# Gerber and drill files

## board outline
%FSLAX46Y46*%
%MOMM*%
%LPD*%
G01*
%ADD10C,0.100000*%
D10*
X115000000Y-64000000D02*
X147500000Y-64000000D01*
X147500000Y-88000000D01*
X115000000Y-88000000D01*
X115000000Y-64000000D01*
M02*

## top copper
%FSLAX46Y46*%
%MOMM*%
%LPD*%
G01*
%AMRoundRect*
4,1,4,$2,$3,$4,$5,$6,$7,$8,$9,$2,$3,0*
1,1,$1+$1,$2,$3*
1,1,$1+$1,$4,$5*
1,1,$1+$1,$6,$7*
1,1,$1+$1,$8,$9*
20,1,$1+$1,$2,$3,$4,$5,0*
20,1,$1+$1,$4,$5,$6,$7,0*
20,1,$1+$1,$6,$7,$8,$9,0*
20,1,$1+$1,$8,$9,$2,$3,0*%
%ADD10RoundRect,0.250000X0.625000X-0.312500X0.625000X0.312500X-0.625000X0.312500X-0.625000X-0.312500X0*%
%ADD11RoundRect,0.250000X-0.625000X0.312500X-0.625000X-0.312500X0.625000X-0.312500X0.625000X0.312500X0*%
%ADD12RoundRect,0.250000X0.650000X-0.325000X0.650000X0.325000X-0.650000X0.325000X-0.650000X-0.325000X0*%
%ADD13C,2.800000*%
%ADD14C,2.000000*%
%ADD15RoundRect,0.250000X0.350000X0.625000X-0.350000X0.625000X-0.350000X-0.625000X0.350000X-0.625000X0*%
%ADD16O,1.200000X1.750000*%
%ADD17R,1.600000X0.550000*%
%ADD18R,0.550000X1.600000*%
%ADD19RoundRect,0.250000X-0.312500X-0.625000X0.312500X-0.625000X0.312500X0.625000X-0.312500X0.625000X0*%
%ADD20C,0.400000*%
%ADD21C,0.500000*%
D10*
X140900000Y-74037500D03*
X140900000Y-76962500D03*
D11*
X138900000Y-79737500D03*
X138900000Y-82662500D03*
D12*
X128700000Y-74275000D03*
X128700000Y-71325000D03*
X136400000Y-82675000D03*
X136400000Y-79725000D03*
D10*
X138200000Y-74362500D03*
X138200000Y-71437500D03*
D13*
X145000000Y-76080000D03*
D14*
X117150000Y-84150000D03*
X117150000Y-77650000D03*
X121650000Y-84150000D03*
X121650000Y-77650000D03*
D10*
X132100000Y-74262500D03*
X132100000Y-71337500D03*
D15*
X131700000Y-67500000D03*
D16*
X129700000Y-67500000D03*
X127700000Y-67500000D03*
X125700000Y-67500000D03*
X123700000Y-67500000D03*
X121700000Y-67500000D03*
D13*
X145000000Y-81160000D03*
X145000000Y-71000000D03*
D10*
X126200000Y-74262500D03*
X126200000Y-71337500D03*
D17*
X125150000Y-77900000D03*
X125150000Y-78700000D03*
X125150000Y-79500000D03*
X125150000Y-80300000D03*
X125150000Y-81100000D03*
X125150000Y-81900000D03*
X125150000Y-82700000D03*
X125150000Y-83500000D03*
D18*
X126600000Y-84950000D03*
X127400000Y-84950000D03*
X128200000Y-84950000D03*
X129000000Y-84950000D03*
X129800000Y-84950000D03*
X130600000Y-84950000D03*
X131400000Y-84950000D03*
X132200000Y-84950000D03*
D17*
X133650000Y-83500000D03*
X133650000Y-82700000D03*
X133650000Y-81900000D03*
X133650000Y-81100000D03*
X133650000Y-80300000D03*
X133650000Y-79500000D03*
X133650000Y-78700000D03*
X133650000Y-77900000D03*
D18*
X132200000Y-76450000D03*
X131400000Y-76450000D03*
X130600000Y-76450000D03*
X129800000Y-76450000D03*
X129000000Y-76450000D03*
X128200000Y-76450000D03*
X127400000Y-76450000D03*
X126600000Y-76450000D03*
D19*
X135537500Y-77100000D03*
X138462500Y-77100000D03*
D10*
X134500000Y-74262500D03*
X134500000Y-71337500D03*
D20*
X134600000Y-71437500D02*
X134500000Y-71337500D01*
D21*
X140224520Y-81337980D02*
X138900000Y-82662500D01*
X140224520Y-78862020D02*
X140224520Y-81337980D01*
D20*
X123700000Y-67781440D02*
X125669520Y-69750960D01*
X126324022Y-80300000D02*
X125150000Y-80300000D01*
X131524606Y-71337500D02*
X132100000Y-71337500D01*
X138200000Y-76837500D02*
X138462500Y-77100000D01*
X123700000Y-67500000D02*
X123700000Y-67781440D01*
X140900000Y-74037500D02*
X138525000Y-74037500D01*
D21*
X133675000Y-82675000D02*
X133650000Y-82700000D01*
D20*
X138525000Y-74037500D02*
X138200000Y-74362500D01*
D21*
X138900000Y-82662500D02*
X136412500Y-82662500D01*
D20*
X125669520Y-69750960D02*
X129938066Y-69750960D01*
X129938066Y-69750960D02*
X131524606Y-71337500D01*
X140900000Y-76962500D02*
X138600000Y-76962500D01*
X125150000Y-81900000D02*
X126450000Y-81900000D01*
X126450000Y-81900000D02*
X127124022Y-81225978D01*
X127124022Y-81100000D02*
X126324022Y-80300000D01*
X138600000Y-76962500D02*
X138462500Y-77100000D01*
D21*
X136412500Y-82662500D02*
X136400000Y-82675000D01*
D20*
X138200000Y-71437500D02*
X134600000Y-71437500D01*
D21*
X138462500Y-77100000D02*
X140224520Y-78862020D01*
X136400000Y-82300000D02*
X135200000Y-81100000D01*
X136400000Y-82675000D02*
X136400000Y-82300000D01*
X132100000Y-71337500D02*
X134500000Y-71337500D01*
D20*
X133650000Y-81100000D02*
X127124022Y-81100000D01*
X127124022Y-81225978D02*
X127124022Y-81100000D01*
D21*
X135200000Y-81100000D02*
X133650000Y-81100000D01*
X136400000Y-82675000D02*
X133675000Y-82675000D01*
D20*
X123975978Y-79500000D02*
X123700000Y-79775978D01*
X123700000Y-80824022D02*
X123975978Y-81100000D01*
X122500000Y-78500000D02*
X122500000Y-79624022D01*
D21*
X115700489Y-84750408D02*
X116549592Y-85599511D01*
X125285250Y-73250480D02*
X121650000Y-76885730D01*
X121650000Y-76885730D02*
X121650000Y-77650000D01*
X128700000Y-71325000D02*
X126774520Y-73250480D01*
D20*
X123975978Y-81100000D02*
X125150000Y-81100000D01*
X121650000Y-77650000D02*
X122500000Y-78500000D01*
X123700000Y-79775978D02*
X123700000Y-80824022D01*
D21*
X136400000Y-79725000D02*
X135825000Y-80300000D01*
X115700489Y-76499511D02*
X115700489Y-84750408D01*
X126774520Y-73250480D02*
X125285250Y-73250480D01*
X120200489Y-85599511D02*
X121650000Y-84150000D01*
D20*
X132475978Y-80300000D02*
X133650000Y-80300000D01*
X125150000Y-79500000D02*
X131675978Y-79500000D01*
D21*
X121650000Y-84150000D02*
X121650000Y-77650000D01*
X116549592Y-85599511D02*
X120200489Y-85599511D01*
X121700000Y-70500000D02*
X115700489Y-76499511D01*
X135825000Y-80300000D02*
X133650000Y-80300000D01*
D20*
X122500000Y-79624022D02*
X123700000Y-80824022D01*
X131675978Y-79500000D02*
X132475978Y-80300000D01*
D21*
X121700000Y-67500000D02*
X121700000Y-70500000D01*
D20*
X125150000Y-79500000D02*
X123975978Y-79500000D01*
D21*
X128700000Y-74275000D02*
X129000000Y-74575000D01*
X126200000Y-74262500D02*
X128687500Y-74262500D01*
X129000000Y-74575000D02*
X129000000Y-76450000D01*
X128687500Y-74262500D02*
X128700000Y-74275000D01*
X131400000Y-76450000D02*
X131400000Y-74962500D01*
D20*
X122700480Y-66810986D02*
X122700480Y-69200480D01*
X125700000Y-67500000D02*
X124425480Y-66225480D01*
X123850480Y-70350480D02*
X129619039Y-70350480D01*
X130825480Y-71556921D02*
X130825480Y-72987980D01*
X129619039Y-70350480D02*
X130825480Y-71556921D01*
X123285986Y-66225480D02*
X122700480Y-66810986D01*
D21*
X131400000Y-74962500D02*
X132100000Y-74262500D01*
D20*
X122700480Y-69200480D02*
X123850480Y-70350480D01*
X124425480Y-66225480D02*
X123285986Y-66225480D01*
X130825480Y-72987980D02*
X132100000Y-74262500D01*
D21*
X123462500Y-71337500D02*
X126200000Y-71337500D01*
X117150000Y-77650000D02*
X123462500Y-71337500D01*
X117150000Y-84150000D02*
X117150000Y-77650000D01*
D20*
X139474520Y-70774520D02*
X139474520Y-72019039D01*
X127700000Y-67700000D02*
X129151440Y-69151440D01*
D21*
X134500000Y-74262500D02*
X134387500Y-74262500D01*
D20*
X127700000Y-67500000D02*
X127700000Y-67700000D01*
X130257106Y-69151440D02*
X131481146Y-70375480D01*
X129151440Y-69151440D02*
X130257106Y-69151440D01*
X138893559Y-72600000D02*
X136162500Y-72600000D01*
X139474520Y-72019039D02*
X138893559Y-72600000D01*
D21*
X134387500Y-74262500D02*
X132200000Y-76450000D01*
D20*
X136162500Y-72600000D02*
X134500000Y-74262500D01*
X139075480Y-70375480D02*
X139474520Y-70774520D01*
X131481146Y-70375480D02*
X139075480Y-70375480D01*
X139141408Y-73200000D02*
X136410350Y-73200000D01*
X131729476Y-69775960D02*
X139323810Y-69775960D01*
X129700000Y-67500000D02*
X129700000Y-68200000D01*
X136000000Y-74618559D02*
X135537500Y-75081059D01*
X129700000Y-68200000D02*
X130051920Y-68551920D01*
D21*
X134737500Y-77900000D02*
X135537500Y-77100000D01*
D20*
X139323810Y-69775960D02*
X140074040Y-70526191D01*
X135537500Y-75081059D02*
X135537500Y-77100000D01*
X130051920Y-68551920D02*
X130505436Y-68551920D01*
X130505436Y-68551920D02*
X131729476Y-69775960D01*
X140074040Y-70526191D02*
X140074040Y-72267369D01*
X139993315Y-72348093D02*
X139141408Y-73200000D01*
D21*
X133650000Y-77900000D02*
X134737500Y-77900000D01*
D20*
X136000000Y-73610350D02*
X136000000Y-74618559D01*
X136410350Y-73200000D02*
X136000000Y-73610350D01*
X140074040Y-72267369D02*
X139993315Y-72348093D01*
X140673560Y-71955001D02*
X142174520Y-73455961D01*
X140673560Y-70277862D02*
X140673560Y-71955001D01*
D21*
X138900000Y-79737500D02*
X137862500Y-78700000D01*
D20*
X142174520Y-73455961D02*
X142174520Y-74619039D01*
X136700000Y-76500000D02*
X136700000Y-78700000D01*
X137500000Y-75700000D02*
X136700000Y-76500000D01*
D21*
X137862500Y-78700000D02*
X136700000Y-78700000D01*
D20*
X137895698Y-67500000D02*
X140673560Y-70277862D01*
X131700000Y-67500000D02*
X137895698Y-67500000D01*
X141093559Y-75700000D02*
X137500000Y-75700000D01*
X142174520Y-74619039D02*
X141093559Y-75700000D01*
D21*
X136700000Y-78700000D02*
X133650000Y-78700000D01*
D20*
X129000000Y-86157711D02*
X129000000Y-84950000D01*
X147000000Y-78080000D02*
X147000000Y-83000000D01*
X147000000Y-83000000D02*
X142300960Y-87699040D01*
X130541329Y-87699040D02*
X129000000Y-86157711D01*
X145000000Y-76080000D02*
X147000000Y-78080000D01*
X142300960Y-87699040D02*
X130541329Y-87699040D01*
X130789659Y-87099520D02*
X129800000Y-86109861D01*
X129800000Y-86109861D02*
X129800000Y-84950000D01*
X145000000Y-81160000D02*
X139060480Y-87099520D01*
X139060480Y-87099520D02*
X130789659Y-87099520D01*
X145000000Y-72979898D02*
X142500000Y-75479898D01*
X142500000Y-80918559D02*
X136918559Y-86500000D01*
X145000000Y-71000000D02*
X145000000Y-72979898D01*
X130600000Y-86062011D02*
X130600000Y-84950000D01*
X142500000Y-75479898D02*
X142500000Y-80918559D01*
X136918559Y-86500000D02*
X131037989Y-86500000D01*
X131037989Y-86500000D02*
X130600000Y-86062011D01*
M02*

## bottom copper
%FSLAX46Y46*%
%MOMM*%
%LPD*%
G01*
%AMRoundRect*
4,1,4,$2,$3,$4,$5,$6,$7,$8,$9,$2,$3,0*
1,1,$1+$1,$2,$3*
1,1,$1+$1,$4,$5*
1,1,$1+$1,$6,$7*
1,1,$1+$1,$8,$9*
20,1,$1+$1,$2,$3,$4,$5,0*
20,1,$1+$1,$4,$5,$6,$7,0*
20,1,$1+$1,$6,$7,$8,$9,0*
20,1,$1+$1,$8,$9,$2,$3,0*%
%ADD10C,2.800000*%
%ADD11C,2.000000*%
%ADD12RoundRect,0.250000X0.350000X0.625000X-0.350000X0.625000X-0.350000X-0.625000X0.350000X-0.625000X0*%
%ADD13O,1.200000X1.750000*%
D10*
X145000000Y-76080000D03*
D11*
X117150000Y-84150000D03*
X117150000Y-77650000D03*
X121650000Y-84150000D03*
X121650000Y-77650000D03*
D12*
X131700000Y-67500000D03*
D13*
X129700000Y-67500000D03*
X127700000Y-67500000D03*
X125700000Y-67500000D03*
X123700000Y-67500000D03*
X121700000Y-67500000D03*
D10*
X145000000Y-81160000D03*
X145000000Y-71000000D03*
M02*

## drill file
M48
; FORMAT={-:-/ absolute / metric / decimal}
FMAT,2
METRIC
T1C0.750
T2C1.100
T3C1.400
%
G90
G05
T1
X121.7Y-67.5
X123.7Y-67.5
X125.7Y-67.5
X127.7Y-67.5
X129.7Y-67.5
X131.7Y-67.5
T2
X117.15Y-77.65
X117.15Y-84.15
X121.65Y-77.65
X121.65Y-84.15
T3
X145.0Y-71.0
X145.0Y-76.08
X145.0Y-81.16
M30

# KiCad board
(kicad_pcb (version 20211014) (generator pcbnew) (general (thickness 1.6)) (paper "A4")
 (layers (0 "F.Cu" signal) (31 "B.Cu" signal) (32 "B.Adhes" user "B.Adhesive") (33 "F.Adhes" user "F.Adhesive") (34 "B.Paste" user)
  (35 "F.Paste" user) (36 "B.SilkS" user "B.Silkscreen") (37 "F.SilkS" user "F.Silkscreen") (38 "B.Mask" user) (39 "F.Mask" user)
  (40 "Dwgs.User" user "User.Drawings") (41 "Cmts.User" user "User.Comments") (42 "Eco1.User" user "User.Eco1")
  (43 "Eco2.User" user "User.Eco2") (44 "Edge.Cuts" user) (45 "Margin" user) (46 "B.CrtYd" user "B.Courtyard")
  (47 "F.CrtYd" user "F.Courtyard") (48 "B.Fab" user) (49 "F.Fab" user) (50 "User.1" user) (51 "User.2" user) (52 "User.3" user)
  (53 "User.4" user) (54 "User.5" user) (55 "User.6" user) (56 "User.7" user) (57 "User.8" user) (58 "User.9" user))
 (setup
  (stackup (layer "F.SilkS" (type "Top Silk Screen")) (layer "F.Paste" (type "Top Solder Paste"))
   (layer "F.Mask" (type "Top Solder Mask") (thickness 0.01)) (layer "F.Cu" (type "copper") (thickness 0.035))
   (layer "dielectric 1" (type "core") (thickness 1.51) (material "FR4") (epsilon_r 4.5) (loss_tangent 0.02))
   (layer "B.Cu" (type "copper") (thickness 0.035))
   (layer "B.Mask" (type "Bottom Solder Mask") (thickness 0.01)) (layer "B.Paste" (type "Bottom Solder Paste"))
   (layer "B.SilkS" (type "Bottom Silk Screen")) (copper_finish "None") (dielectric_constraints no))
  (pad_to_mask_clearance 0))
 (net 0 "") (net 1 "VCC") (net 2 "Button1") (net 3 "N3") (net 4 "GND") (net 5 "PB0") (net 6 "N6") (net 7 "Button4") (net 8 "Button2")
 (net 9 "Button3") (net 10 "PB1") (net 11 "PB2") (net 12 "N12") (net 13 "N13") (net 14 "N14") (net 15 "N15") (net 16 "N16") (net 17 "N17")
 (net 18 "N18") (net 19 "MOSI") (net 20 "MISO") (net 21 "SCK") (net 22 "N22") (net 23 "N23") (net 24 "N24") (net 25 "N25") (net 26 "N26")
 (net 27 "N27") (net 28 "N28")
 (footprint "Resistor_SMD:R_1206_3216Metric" (layer "F.Cu") (at 140.9 75.5 90)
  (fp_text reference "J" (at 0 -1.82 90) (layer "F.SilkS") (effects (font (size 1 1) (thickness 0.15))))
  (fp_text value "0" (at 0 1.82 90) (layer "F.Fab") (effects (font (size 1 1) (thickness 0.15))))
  (pad "1" smd roundrect (at 1.4625 0 90) (size 1.125 1.75) (layers "F.Cu" "F.Paste" "F.Mask") (roundrect_rratio 0.2222222222) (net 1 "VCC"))
  (pad "1" smd roundrect (at -1.4625 0 90) (size 1.125 1.75) (layers "F.Cu" "F.Paste" "F.Mask") (roundrect_rratio 0.2222222222)
   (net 1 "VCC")))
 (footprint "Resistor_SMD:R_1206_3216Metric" (layer "F.Cu") (at 138.9 81.2 -90)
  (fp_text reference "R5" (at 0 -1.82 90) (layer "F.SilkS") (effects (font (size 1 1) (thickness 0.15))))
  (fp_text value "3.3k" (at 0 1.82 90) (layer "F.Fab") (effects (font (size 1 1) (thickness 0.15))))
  (pad "1" smd roundrect (at -1.4625 0 270) (size 1.125 1.75) (layers "F.Cu" "F.Paste" "F.Mask") (roundrect_rratio 0.2222222222)
   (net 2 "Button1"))
  (pad "2" smd roundrect (at 1.4625 0 270) (size 1.125 1.75) (layers "F.Cu" "F.Paste" "F.Mask") (roundrect_rratio 0.2222222222)
   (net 1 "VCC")))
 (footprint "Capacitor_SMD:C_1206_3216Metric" (layer "F.Cu") (at 128.7 72.8 90)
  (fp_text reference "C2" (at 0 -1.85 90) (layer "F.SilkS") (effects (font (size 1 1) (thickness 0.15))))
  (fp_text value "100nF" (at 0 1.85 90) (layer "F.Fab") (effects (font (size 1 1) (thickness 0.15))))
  (pad "1" smd roundrect (at -1.475 0 90) (size 1.15 1.8) (layers "F.Cu" "F.Paste" "F.Mask") (roundrect_rratio 0.2173913043) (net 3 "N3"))
  (pad "2" smd roundrect (at 1.475 0 90) (size 1.15 1.8) (layers "F.Cu" "F.Paste" "F.Mask") (roundrect_rratio 0.2173913043) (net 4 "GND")))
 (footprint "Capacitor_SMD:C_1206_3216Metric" (layer "F.Cu") (at 136.4 81.2 90)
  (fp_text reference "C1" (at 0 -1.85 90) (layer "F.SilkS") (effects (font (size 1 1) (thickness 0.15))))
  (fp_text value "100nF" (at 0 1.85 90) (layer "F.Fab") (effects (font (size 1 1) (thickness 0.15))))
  (pad "1" smd roundrect (at -1.475 0 90) (size 1.15 1.8) (layers "F.Cu" "F.Paste" "F.Mask") (roundrect_rratio 0.2173913043) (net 1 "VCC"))
  (pad "2" smd roundrect (at 1.475 0 90) (size 1.15 1.8) (layers "F.Cu" "F.Paste" "F.Mask") (roundrect_rratio 0.2173913043) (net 4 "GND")))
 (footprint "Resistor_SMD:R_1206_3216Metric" (layer "F.Cu") (at 138.2 72.9 90)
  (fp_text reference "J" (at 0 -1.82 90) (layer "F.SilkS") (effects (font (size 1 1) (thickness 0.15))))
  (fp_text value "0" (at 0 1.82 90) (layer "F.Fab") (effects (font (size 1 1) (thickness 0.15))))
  (pad "1" smd roundrect (at -1.4625 0 90) (size 1.125 1.75) (layers "F.Cu" "F.Paste" "F.Mask") (roundrect_rratio 0.2222222222)
   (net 1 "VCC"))
  (pad "1" smd roundrect (at 1.4625 0 90) (size 1.125 1.75) (layers "F.Cu" "F.Paste" "F.Mask") (roundrect_rratio 0.2222222222) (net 1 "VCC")))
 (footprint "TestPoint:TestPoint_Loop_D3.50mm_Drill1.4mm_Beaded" (layer "F.Cu") (at 145 76.08)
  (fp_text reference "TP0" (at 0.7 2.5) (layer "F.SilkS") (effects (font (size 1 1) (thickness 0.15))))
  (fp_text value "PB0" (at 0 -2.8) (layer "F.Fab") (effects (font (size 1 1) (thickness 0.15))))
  (pad "1" thru_hole circle (at 0 0) (size 2.8 2.8) (drill 1.4) (layers *.Cu *.Mask) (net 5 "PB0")))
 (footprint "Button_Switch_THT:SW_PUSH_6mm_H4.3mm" (layer "F.Cu") (at 117.15 84.15 90)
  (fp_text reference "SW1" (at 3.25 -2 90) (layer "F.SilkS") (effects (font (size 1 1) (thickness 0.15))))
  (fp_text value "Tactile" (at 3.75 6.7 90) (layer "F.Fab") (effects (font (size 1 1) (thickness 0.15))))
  (pad "1" thru_hole circle (at 0 0 180) (size 2 2) (drill 1.1) (layers *.Cu *.Mask) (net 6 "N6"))
  (pad "1" thru_hole circle (at 6.5 0 180) (size 2 2) (drill 1.1) (layers *.Cu *.Mask) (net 6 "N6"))
  (pad "2" thru_hole circle (at 0 4.5 180) (size 2 2) (drill 1.1) (layers *.Cu *.Mask) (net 4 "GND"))
  (pad "2" thru_hole circle (at 6.5 4.5 180) (size 2 2) (drill 1.1) (layers *.Cu *.Mask) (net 4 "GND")))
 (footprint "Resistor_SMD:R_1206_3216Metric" (layer "F.Cu") (at 132.1 72.8 90)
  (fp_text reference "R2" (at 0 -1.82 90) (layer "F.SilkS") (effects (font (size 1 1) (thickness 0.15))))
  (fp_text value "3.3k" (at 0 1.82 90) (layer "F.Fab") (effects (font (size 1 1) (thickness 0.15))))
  (pad "1" smd roundrect (at -1.4625 0 90) (size 1.125 1.75) (layers "F.Cu" "F.Paste" "F.Mask") (roundrect_rratio 0.2222222222)
   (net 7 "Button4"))
  (pad "2" smd roundrect (at 1.4625 0 90) (size 1.125 1.75) (layers "F.Cu" "F.Paste" "F.Mask") (roundrect_rratio 0.2222222222) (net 1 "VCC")))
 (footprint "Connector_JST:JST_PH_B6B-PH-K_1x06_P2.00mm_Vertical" (layer "F.Cu") (at 131.7 67.5 180)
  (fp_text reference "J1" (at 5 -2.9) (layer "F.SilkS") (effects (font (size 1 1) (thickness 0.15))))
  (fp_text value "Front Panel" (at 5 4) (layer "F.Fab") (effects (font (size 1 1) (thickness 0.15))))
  (pad "1" thru_hole roundrect (at 0 0 180) (size 1.2 1.75) (drill 0.75) (layers *.Cu *.Mask) (roundrect_rratio 0.2083333333)
   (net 2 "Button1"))
  (pad "2" thru_hole oval (at 2 0 180) (size 1.2 1.75) (drill 0.75) (layers *.Cu *.Mask) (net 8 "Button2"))
  (pad "3" thru_hole oval (at 4 0 180) (size 1.2 1.75) (drill 0.75) (layers *.Cu *.Mask) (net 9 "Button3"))
  (pad "4" thru_hole oval (at 6 0 180) (size 1.2 1.75) (drill 0.75) (layers *.Cu *.Mask) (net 7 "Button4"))
  (pad "5" thru_hole oval (at 8 0 180) (size 1.2 1.75) (drill 0.75) (layers *.Cu *.Mask) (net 1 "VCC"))
  (pad "6" thru_hole oval (at 10 0 180) (size 1.2 1.75) (drill 0.75) (layers *.Cu *.Mask) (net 4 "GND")))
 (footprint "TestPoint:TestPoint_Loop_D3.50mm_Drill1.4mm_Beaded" (layer "F.Cu") (at 145 81.16)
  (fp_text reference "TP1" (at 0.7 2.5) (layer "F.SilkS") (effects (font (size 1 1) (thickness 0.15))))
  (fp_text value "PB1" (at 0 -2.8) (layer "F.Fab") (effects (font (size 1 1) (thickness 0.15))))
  (pad "1" thru_hole circle (at 0 0) (size 2.8 2.8) (drill 1.4) (layers *.Cu *.Mask) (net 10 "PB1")))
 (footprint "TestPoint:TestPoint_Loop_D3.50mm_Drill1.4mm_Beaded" (layer "F.Cu") (at 145 71)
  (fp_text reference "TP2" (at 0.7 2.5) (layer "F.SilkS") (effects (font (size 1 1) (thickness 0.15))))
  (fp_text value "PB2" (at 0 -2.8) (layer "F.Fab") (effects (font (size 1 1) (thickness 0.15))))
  (pad "1" thru_hole circle (at 0 0) (size 2.8 2.8) (drill 1.4) (layers *.Cu *.Mask) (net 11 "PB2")))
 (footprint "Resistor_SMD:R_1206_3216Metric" (layer "F.Cu") (at 126.2 72.8 90)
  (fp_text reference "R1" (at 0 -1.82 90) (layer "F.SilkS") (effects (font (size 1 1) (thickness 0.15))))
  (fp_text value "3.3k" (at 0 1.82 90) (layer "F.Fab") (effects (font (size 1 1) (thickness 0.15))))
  (pad "1" smd roundrect (at -1.4625 0 90) (size 1.125 1.75) (layers "F.Cu" "F.Paste" "F.Mask") (roundrect_rratio 0.2222222222) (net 3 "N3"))
  (pad "2" smd roundrect (at 1.4625 0 90) (size 1.125 1.75) (layers "F.Cu" "F.Paste" "F.Mask") (roundrect_rratio 0.2222222222) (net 6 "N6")))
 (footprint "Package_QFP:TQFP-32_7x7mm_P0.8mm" (layer "F.Cu") (at 129.4 80.7)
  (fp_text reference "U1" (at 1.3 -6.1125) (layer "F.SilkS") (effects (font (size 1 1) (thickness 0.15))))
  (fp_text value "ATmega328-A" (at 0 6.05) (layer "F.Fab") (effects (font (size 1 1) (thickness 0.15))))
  (pad "1" smd rect (at -4.25 -2.8) (size 1.6 0.55) (layers "F.Cu" "F.Paste" "F.Mask") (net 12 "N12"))
  (pad "2" smd rect (at -4.25 -2) (size 1.6 0.55) (layers "F.Cu" "F.Paste" "F.Mask") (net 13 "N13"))
  (pad "3" smd rect (at -4.25 -1.2) (size 1.6 0.55) (layers "F.Cu" "F.Paste" "F.Mask") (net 4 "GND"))
  (pad "4" smd rect (at -4.25 -0.4) (size 1.6 0.55) (layers "F.Cu" "F.Paste" "F.Mask") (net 1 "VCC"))
  (pad "5" smd rect (at -4.25 0.4) (size 1.6 0.55) (layers "F.Cu" "F.Paste" "F.Mask") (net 4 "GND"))
  (pad "6" smd rect (at -4.25 1.2) (size 1.6 0.55) (layers "F.Cu" "F.Paste" "F.Mask") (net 1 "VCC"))
  (pad "7" smd rect (at -4.25 2) (size 1.6 0.55) (layers "F.Cu" "F.Paste" "F.Mask") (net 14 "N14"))
  (pad "8" smd rect (at -4.25 2.8) (size 1.6 0.55) (layers "F.Cu" "F.Paste" "F.Mask") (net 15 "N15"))
  (pad "9" smd rect (at -2.8 4.25 90) (size 1.6 0.55) (layers "F.Cu" "F.Paste" "F.Mask") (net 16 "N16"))
  (pad "10" smd rect (at -2 4.25 90) (size 1.6 0.55) (layers "F.Cu" "F.Paste" "F.Mask") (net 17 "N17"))
  (pad "11" smd rect (at -1.2 4.25 90) (size 1.6 0.55) (layers "F.Cu" "F.Paste" "F.Mask") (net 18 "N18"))
  (pad "12" smd rect (at -0.4 4.25 90) (size 1.6 0.55) (layers "F.Cu" "F.Paste" "F.Mask") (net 5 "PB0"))
  (pad "13" smd rect (at 0.4 4.25 90) (size 1.6 0.55) (layers "F.Cu" "F.Paste" "F.Mask") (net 10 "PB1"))
  (pad "14" smd rect (at 1.2 4.25 90) (size 1.6 0.55) (layers "F.Cu" "F.Paste" "F.Mask") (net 11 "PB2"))
  (pad "15" smd rect (at 2 4.25 90) (size 1.6 0.55) (layers "F.Cu" "F.Paste" "F.Mask") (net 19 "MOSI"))
  (pad "16" smd rect (at 2.8 4.25 90) (size 1.6 0.55) (layers "F.Cu" "F.Paste" "F.Mask") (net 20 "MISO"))
  (pad "17" smd rect (at 4.25 2.8) (size 1.6 0.55) (layers "F.Cu" "F.Paste" "F.Mask") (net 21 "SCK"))
  (pad "18" smd rect (at 4.25 2) (size 1.6 0.55) (layers "F.Cu" "F.Paste" "F.Mask") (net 1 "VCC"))
  (pad "19" smd rect (at 4.25 1.2) (size 1.6 0.55) (layers "F.Cu" "F.Paste" "F.Mask") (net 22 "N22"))
  (pad "20" smd rect (at 4.25 0.4) (size 1.6 0.55) (layers "F.Cu" "F.Paste" "F.Mask") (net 1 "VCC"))
  (pad "21" smd rect (at 4.25 -0.4) (size 1.6 0.55) (layers "F.Cu" "F.Paste" "F.Mask") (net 4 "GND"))
  (pad "22" smd rect (at 4.25 -1.2) (size 1.6 0.55) (layers "F.Cu" "F.Paste" "F.Mask") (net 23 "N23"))
  (pad "23" smd rect (at 4.25 -2) (size 1.6 0.55) (layers "F.Cu" "F.Paste" "F.Mask") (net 2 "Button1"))
  (pad "24" smd rect (at 4.25 -2.8) (size 1.6 0.55) (layers "F.Cu" "F.Paste" "F.Mask") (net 8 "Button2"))
  (pad "25" smd rect (at 2.8 -4.25 90) (size 1.6 0.55) (layers "F.Cu" "F.Paste" "F.Mask") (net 9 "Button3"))
  (pad "26" smd rect (at 2 -4.25 90) (size 1.6 0.55) (layers "F.Cu" "F.Paste" "F.Mask") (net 7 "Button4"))
  (pad "27" smd rect (at 1.2 -4.25 90) (size 1.6 0.55) (layers "F.Cu" "F.Paste" "F.Mask") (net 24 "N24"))
  (pad "28" smd rect (at 0.4 -4.25 90) (size 1.6 0.55) (layers "F.Cu" "F.Paste" "F.Mask") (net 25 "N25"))
  (pad "29" smd rect (at -0.4 -4.25 90) (size 1.6 0.55) (layers "F.Cu" "F.Paste" "F.Mask") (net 3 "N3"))
  (pad "30" smd rect (at -1.2 -4.25 90) (size 1.6 0.55) (layers "F.Cu" "F.Paste" "F.Mask") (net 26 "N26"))
  (pad "31" smd rect (at -2 -4.25 90) (size 1.6 0.55) (layers "F.Cu" "F.Paste" "F.Mask") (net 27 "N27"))
  (pad "32" smd rect (at -2.8 -4.25 90) (size 1.6 0.55) (layers "F.Cu" "F.Paste" "F.Mask") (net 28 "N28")))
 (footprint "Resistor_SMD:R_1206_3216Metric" (layer "F.Cu") (at 137 77.1)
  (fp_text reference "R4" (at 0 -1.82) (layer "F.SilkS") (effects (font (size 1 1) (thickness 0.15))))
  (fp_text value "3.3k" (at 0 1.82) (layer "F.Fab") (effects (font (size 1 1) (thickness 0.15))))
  (pad "1" smd roundrect (at -1.4625 0) (size 1.125 1.75) (layers "F.Cu" "F.Paste" "F.Mask") (roundrect_rratio 0.2222222222)
   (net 8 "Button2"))
  (pad "2" smd roundrect (at 1.4625 0) (size 1.125 1.75) (layers "F.Cu" "F.Paste" "F.Mask") (roundrect_rratio 0.2222222222) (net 1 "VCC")))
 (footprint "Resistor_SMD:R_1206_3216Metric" (layer "F.Cu") (at 134.5 72.8 90)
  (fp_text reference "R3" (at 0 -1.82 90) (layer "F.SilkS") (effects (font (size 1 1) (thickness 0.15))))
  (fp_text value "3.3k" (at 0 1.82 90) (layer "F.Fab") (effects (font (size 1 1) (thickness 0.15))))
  (pad "1" smd roundrect (at -1.4625 0 90) (size 1.125 1.75) (layers "F.Cu" "F.Paste" "F.Mask") (roundrect_rratio 0.2222222222)
   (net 9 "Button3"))
  (pad "2" smd roundrect (at 1.4625 0 90) (size 1.125 1.75) (layers "F.Cu" "F.Paste" "F.Mask") (roundrect_rratio 0.2222222222) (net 1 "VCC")))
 (gr_rect (start 115 64) (end 147.5 88) (layer "Edge.Cuts") (width 0.1) (fill none))
 (segment (start 134.6 71.4375) (end 134.5 71.3375) (width 0.4) (layer "F.Cu") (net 1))
 (segment (start 140.22452 81.33798) (end 138.9 82.6625) (width 0.5) (layer "F.Cu") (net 1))
 (segment (start 140.22452 78.86202) (end 140.22452 81.33798) (width 0.5) (layer "F.Cu") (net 1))
 (segment (start 123.7 67.78144) (end 125.66952 69.75096) (width 0.4) (layer "F.Cu") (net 1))
 (segment (start 126.324022 80.3) (end 125.15 80.3) (width 0.4) (layer "F.Cu") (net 1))
 (segment (start 131.524606 71.3375) (end 132.1 71.3375) (width 0.4) (layer "F.Cu") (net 1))
 (segment (start 138.2 76.8375) (end 138.4625 77.1) (width 0.4) (layer "F.Cu") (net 1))
 (segment (start 123.7 67.5) (end 123.7 67.78144) (width 0.4) (layer "F.Cu") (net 1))
 (segment (start 140.9 74.0375) (end 138.525 74.0375) (width 0.4) (layer "F.Cu") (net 1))
 (segment (start 133.675 82.675) (end 133.65 82.7) (width 0.5) (layer "F.Cu") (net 1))
 (segment (start 138.525 74.0375) (end 138.2 74.3625) (width 0.4) (layer "F.Cu") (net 1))
 (segment (start 138.9 82.6625) (end 136.4125 82.6625) (width 0.5) (layer "F.Cu") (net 1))
 (segment (start 125.66952 69.75096) (end 129.938066 69.75096) (width 0.4) (layer "F.Cu") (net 1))
 (segment (start 129.938066 69.75096) (end 131.524606 71.3375) (width 0.4) (layer "F.Cu") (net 1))
 (segment (start 140.9 76.9625) (end 138.6 76.9625) (width 0.4) (layer "F.Cu") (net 1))
 (segment (start 125.15 81.9) (end 126.45 81.9) (width 0.4) (layer "F.Cu") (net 1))
 (segment (start 126.45 81.9) (end 127.124022 81.225978) (width 0.4) (layer "F.Cu") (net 1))
 (segment (start 127.124022 81.1) (end 126.324022 80.3) (width 0.4) (layer "F.Cu") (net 1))
 (segment (start 138.6 76.9625) (end 138.4625 77.1) (width 0.4) (layer "F.Cu") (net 1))
 (segment (start 136.4125 82.6625) (end 136.4 82.675) (width 0.5) (layer "F.Cu") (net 1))
 (segment (start 138.2 71.4375) (end 134.6 71.4375) (width 0.4) (layer "F.Cu") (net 1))
 (segment (start 138.4625 77.1) (end 140.22452 78.86202) (width 0.5) (layer "F.Cu") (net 1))
 (segment (start 136.4 82.3) (end 135.2 81.1) (width 0.5) (layer "F.Cu") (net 1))
 (segment (start 136.4 82.675) (end 136.4 82.3) (width 0.5) (layer "F.Cu") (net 1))
 (segment (start 132.1 71.3375) (end 134.5 71.3375) (width 0.5) (layer "F.Cu") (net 1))
 (segment (start 133.65 81.1) (end 127.124022 81.1) (width 0.4) (layer "F.Cu") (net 1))
 (segment (start 127.124022 81.225978) (end 127.124022 81.1) (width 0.4) (layer "F.Cu") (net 1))
 (segment (start 135.2 81.1) (end 133.65 81.1) (width 0.5) (layer "F.Cu") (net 1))
 (segment (start 136.4 82.675) (end 133.675 82.675) (width 0.5) (layer "F.Cu") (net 1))
 (segment (start 123.975978 79.5) (end 123.7 79.775978) (width 0.4) (layer "F.Cu") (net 4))
 (segment (start 123.7 80.824022) (end 123.975978 81.1) (width 0.4) (layer "F.Cu") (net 4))
 (segment (start 122.5 78.5) (end 122.5 79.624022) (width 0.4) (layer "F.Cu") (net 4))
 (segment (start 115.700489 84.750408) (end 116.549592 85.599511) (width 0.5) (layer "F.Cu") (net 4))
 (segment (start 125.28525 73.25048) (end 121.65 76.88573) (width 0.5) (layer "F.Cu") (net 4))
 (segment (start 121.65 76.88573) (end 121.65 77.65) (width 0.5) (layer "F.Cu") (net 4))
 (segment (start 128.7 71.325) (end 126.77452 73.25048) (width 0.5) (layer "F.Cu") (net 4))
 (segment (start 123.975978 81.1) (end 125.15 81.1) (width 0.4) (layer "F.Cu") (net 4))
 (segment (start 121.65 77.65) (end 122.5 78.5) (width 0.4) (layer "F.Cu") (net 4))
 (segment (start 123.7 79.775978) (end 123.7 80.824022) (width 0.4) (layer "F.Cu") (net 4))
 (segment (start 136.4 79.725) (end 135.825 80.3) (width 0.5) (layer "F.Cu") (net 4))
 (segment (start 115.700489 76.499511) (end 115.700489 84.750408) (width 0.5) (layer "F.Cu") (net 4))
 (segment (start 126.77452 73.25048) (end 125.28525 73.25048) (width 0.5) (layer "F.Cu") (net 4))
 (segment (start 120.200489 85.599511) (end 121.65 84.15) (width 0.5) (layer "F.Cu") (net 4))
 (segment (start 132.475978 80.3) (end 133.65 80.3) (width 0.4) (layer "F.Cu") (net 4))
 (segment (start 125.15 79.5) (end 131.675978 79.5) (width 0.4) (layer "F.Cu") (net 4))
 (segment (start 121.65 84.15) (end 121.65 77.65) (width 0.5) (layer "F.Cu") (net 4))
 (segment (start 116.549592 85.599511) (end 120.200489 85.599511) (width 0.5) (layer "F.Cu") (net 4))
 (segment (start 121.7 70.5) (end 115.700489 76.499511) (width 0.5) (layer "F.Cu") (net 4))
 (segment (start 135.825 80.3) (end 133.65 80.3) (width 0.5) (layer "F.Cu") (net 4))
 (segment (start 122.5 79.624022) (end 123.7 80.824022) (width 0.4) (layer "F.Cu") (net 4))
 (segment (start 131.675978 79.5) (end 132.475978 80.3) (width 0.4) (layer "F.Cu") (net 4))
 (segment (start 121.7 67.5) (end 121.7 70.5) (width 0.5) (layer "F.Cu") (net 4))
 (segment (start 125.15 79.5) (end 123.975978 79.5) (width 0.4) (layer "F.Cu") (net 4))
 (segment (start 128.7 74.275) (end 129 74.575) (width 0.5) (layer "F.Cu") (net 3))
 (segment (start 126.2 74.2625) (end 128.6875 74.2625) (width 0.5) (layer "F.Cu") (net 3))
 (segment (start 129 74.575) (end 129 76.45) (width 0.5) (layer "F.Cu") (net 3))
 (segment (start 128.6875 74.2625) (end 128.7 74.275) (width 0.5) (layer "F.Cu") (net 3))
 (segment (start 131.4 76.45) (end 131.4 74.9625) (width 0.5) (layer "F.Cu") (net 7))
 (segment (start 122.70048 66.810986) (end 122.70048 69.20048) (width 0.4) (layer "F.Cu") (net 7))
 (segment (start 125.7 67.5) (end 124.42548 66.22548) (width 0.4) (layer "F.Cu") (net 7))
 (segment (start 123.85048 70.35048) (end 129.619039 70.35048) (width 0.4) (layer "F.Cu") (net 7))
 (segment (start 130.82548 71.556921) (end 130.82548 72.98798) (width 0.4) (layer "F.Cu") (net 7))
 (segment (start 129.619039 70.35048) (end 130.82548 71.556921) (width 0.4) (layer "F.Cu") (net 7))
 (segment (start 123.285986 66.22548) (end 122.70048 66.810986) (width 0.4) (layer "F.Cu") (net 7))
 (segment (start 131.4 74.9625) (end 132.1 74.2625) (width 0.5) (layer "F.Cu") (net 7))
 (segment (start 122.70048 69.20048) (end 123.85048 70.35048) (width 0.4) (layer "F.Cu") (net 7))
 (segment (start 124.42548 66.22548) (end 123.285986 66.22548) (width 0.4) (layer "F.Cu") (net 7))
 (segment (start 130.82548 72.98798) (end 132.1 74.2625) (width 0.4) (layer "F.Cu") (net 7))
 (segment (start 123.4625 71.3375) (end 126.2 71.3375) (width 0.5) (layer "F.Cu") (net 6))
 (segment (start 117.15 77.65) (end 123.4625 71.3375) (width 0.5) (layer "F.Cu") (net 6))
 (segment (start 117.15 84.15) (end 117.15 77.65) (width 0.5) (layer "F.Cu") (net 6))
 (segment (start 139.47452 70.77452) (end 139.47452 72.019039) (width 0.4) (layer "F.Cu") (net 9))
 (segment (start 127.7 67.7) (end 129.15144 69.15144) (width 0.4) (layer "F.Cu") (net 9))
 (segment (start 134.5 74.2625) (end 134.3875 74.2625) (width 0.5) (layer "F.Cu") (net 9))
 (segment (start 127.7 67.5) (end 127.7 67.7) (width 0.4) (layer "F.Cu") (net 9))
 (segment (start 130.257106 69.15144) (end 131.481146 70.37548) (width 0.4) (layer "F.Cu") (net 9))
 (segment (start 129.15144 69.15144) (end 130.257106 69.15144) (width 0.4) (layer "F.Cu") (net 9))
 (segment (start 138.893559 72.6) (end 136.1625 72.6) (width 0.4) (layer "F.Cu") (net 9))
 (segment (start 139.47452 72.019039) (end 138.893559 72.6) (width 0.4) (layer "F.Cu") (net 9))
 (segment (start 134.3875 74.2625) (end 132.2 76.45) (width 0.5) (layer "F.Cu") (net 9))
 (segment (start 136.1625 72.6) (end 134.5 74.2625) (width 0.4) (layer "F.Cu") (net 9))
 (segment (start 139.07548 70.37548) (end 139.47452 70.77452) (width 0.4) (layer "F.Cu") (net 9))
 (segment (start 131.481146 70.37548) (end 139.07548 70.37548) (width 0.4) (layer "F.Cu") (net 9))
 (segment (start 139.141408 73.2) (end 136.41035 73.2) (width 0.4) (layer "F.Cu") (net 8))
 (segment (start 131.729476 69.77596) (end 139.32381 69.77596) (width 0.4) (layer "F.Cu") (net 8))
 (segment (start 129.7 67.5) (end 129.7 68.2) (width 0.4) (layer "F.Cu") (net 8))
 (segment (start 136 74.618559) (end 135.5375 75.081059) (width 0.4) (layer "F.Cu") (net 8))
 (segment (start 129.7 68.2) (end 130.05192 68.55192) (width 0.4) (layer "F.Cu") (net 8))
 (segment (start 134.7375 77.9) (end 135.5375 77.1) (width 0.5) (layer "F.Cu") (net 8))
 (segment (start 139.32381 69.77596) (end 140.07404 70.526191) (width 0.4) (layer "F.Cu") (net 8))
 (segment (start 135.5375 75.081059) (end 135.5375 77.1) (width 0.4) (layer "F.Cu") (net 8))
 (segment (start 130.05192 68.55192) (end 130.505436 68.55192) (width 0.4) (layer "F.Cu") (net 8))
 (segment (start 130.505436 68.55192) (end 131.729476 69.77596) (width 0.4) (layer "F.Cu") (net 8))
 (segment (start 140.07404 70.526191) (end 140.07404 72.267369) (width 0.4) (layer "F.Cu") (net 8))
 (segment (start 139.993315 72.348093) (end 139.141408 73.2) (width 0.4) (layer "F.Cu") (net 8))
 (segment (start 133.65 77.9) (end 134.7375 77.9) (width 0.5) (layer "F.Cu") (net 8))
 (segment (start 136 73.61035) (end 136 74.618559) (width 0.4) (layer "F.Cu") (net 8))
 (segment (start 136.41035 73.2) (end 136 73.61035) (width 0.4) (layer "F.Cu") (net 8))
 (segment (start 140.07404 72.267369) (end 139.993315 72.348093) (width 0.4) (layer "F.Cu") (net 8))
 (segment (start 140.67356 71.955001) (end 142.17452 73.455961) (width 0.4) (layer "F.Cu") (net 2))
 (segment (start 140.67356 70.277862) (end 140.67356 71.955001) (width 0.4) (layer "F.Cu") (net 2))
 (segment (start 138.9 79.7375) (end 137.8625 78.7) (width 0.5) (layer "F.Cu") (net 2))
 (segment (start 142.17452 73.455961) (end 142.17452 74.619039) (width 0.4) (layer "F.Cu") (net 2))
 (segment (start 136.7 76.5) (end 136.7 78.7) (width 0.4) (layer "F.Cu") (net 2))
 (segment (start 137.5 75.7) (end 136.7 76.5) (width 0.4) (layer "F.Cu") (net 2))
 (segment (start 137.8625 78.7) (end 136.7 78.7) (width 0.5) (layer "F.Cu") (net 2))
 (segment (start 137.895698 67.5) (end 140.67356 70.277862) (width 0.4) (layer "F.Cu") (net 2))
 (segment (start 131.7 67.5) (end 137.895698 67.5) (width 0.4) (layer "F.Cu") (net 2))
 (segment (start 141.093559 75.7) (end 137.5 75.7) (width 0.4) (layer "F.Cu") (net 2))
 (segment (start 142.17452 74.619039) (end 141.093559 75.7) (width 0.4) (layer "F.Cu") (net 2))
 (segment (start 136.7 78.7) (end 133.65 78.7) (width 0.5) (layer "F.Cu") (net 2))
 (segment (start 129 86.157711) (end 129 84.95) (width 0.4) (layer "F.Cu") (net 5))
 (segment (start 147 78.08) (end 147 83) (width 0.4) (layer "F.Cu") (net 5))
 (segment (start 147 83) (end 142.30096 87.69904) (width 0.4) (layer "F.Cu") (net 5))
 (segment (start 130.541329 87.69904) (end 129 86.157711) (width 0.4) (layer "F.Cu") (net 5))
 (segment (start 145 76.08) (end 147 78.08) (width 0.4) (layer "F.Cu") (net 5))
 (segment (start 142.30096 87.69904) (end 130.541329 87.69904) (width 0.4) (layer "F.Cu") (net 5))
 (segment (start 130.789659 87.09952) (end 129.8 86.109861) (width 0.4) (layer "F.Cu") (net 10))
 (segment (start 129.8 86.109861) (end 129.8 84.95) (width 0.4) (layer "F.Cu") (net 10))
 (segment (start 145 81.16) (end 139.06048 87.09952) (width 0.4) (layer "F.Cu") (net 10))
 (segment (start 139.06048 87.09952) (end 130.789659 87.09952) (width 0.4) (layer "F.Cu") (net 10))
 (segment (start 145 72.979898) (end 142.5 75.479898) (width 0.4) (layer "F.Cu") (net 11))
 (segment (start 142.5 80.918559) (end 136.918559 86.5) (width 0.4) (layer "F.Cu") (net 11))
 (segment (start 145 71) (end 145 72.979898) (width 0.4) (layer "F.Cu") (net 11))
 (segment (start 130.6 86.062011) (end 130.6 84.95) (width 0.4) (layer "F.Cu") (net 11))
 (segment (start 142.5 75.479898) (end 142.5 80.918559) (width 0.4) (layer "F.Cu") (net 11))
 (segment (start 136.918559 86.5) (end 131.037989 86.5) (width 0.4) (layer "F.Cu") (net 11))
 (segment (start 131.037989 86.5) (end 130.6 86.062011) (width 0.4) (layer "F.Cu") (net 11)))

